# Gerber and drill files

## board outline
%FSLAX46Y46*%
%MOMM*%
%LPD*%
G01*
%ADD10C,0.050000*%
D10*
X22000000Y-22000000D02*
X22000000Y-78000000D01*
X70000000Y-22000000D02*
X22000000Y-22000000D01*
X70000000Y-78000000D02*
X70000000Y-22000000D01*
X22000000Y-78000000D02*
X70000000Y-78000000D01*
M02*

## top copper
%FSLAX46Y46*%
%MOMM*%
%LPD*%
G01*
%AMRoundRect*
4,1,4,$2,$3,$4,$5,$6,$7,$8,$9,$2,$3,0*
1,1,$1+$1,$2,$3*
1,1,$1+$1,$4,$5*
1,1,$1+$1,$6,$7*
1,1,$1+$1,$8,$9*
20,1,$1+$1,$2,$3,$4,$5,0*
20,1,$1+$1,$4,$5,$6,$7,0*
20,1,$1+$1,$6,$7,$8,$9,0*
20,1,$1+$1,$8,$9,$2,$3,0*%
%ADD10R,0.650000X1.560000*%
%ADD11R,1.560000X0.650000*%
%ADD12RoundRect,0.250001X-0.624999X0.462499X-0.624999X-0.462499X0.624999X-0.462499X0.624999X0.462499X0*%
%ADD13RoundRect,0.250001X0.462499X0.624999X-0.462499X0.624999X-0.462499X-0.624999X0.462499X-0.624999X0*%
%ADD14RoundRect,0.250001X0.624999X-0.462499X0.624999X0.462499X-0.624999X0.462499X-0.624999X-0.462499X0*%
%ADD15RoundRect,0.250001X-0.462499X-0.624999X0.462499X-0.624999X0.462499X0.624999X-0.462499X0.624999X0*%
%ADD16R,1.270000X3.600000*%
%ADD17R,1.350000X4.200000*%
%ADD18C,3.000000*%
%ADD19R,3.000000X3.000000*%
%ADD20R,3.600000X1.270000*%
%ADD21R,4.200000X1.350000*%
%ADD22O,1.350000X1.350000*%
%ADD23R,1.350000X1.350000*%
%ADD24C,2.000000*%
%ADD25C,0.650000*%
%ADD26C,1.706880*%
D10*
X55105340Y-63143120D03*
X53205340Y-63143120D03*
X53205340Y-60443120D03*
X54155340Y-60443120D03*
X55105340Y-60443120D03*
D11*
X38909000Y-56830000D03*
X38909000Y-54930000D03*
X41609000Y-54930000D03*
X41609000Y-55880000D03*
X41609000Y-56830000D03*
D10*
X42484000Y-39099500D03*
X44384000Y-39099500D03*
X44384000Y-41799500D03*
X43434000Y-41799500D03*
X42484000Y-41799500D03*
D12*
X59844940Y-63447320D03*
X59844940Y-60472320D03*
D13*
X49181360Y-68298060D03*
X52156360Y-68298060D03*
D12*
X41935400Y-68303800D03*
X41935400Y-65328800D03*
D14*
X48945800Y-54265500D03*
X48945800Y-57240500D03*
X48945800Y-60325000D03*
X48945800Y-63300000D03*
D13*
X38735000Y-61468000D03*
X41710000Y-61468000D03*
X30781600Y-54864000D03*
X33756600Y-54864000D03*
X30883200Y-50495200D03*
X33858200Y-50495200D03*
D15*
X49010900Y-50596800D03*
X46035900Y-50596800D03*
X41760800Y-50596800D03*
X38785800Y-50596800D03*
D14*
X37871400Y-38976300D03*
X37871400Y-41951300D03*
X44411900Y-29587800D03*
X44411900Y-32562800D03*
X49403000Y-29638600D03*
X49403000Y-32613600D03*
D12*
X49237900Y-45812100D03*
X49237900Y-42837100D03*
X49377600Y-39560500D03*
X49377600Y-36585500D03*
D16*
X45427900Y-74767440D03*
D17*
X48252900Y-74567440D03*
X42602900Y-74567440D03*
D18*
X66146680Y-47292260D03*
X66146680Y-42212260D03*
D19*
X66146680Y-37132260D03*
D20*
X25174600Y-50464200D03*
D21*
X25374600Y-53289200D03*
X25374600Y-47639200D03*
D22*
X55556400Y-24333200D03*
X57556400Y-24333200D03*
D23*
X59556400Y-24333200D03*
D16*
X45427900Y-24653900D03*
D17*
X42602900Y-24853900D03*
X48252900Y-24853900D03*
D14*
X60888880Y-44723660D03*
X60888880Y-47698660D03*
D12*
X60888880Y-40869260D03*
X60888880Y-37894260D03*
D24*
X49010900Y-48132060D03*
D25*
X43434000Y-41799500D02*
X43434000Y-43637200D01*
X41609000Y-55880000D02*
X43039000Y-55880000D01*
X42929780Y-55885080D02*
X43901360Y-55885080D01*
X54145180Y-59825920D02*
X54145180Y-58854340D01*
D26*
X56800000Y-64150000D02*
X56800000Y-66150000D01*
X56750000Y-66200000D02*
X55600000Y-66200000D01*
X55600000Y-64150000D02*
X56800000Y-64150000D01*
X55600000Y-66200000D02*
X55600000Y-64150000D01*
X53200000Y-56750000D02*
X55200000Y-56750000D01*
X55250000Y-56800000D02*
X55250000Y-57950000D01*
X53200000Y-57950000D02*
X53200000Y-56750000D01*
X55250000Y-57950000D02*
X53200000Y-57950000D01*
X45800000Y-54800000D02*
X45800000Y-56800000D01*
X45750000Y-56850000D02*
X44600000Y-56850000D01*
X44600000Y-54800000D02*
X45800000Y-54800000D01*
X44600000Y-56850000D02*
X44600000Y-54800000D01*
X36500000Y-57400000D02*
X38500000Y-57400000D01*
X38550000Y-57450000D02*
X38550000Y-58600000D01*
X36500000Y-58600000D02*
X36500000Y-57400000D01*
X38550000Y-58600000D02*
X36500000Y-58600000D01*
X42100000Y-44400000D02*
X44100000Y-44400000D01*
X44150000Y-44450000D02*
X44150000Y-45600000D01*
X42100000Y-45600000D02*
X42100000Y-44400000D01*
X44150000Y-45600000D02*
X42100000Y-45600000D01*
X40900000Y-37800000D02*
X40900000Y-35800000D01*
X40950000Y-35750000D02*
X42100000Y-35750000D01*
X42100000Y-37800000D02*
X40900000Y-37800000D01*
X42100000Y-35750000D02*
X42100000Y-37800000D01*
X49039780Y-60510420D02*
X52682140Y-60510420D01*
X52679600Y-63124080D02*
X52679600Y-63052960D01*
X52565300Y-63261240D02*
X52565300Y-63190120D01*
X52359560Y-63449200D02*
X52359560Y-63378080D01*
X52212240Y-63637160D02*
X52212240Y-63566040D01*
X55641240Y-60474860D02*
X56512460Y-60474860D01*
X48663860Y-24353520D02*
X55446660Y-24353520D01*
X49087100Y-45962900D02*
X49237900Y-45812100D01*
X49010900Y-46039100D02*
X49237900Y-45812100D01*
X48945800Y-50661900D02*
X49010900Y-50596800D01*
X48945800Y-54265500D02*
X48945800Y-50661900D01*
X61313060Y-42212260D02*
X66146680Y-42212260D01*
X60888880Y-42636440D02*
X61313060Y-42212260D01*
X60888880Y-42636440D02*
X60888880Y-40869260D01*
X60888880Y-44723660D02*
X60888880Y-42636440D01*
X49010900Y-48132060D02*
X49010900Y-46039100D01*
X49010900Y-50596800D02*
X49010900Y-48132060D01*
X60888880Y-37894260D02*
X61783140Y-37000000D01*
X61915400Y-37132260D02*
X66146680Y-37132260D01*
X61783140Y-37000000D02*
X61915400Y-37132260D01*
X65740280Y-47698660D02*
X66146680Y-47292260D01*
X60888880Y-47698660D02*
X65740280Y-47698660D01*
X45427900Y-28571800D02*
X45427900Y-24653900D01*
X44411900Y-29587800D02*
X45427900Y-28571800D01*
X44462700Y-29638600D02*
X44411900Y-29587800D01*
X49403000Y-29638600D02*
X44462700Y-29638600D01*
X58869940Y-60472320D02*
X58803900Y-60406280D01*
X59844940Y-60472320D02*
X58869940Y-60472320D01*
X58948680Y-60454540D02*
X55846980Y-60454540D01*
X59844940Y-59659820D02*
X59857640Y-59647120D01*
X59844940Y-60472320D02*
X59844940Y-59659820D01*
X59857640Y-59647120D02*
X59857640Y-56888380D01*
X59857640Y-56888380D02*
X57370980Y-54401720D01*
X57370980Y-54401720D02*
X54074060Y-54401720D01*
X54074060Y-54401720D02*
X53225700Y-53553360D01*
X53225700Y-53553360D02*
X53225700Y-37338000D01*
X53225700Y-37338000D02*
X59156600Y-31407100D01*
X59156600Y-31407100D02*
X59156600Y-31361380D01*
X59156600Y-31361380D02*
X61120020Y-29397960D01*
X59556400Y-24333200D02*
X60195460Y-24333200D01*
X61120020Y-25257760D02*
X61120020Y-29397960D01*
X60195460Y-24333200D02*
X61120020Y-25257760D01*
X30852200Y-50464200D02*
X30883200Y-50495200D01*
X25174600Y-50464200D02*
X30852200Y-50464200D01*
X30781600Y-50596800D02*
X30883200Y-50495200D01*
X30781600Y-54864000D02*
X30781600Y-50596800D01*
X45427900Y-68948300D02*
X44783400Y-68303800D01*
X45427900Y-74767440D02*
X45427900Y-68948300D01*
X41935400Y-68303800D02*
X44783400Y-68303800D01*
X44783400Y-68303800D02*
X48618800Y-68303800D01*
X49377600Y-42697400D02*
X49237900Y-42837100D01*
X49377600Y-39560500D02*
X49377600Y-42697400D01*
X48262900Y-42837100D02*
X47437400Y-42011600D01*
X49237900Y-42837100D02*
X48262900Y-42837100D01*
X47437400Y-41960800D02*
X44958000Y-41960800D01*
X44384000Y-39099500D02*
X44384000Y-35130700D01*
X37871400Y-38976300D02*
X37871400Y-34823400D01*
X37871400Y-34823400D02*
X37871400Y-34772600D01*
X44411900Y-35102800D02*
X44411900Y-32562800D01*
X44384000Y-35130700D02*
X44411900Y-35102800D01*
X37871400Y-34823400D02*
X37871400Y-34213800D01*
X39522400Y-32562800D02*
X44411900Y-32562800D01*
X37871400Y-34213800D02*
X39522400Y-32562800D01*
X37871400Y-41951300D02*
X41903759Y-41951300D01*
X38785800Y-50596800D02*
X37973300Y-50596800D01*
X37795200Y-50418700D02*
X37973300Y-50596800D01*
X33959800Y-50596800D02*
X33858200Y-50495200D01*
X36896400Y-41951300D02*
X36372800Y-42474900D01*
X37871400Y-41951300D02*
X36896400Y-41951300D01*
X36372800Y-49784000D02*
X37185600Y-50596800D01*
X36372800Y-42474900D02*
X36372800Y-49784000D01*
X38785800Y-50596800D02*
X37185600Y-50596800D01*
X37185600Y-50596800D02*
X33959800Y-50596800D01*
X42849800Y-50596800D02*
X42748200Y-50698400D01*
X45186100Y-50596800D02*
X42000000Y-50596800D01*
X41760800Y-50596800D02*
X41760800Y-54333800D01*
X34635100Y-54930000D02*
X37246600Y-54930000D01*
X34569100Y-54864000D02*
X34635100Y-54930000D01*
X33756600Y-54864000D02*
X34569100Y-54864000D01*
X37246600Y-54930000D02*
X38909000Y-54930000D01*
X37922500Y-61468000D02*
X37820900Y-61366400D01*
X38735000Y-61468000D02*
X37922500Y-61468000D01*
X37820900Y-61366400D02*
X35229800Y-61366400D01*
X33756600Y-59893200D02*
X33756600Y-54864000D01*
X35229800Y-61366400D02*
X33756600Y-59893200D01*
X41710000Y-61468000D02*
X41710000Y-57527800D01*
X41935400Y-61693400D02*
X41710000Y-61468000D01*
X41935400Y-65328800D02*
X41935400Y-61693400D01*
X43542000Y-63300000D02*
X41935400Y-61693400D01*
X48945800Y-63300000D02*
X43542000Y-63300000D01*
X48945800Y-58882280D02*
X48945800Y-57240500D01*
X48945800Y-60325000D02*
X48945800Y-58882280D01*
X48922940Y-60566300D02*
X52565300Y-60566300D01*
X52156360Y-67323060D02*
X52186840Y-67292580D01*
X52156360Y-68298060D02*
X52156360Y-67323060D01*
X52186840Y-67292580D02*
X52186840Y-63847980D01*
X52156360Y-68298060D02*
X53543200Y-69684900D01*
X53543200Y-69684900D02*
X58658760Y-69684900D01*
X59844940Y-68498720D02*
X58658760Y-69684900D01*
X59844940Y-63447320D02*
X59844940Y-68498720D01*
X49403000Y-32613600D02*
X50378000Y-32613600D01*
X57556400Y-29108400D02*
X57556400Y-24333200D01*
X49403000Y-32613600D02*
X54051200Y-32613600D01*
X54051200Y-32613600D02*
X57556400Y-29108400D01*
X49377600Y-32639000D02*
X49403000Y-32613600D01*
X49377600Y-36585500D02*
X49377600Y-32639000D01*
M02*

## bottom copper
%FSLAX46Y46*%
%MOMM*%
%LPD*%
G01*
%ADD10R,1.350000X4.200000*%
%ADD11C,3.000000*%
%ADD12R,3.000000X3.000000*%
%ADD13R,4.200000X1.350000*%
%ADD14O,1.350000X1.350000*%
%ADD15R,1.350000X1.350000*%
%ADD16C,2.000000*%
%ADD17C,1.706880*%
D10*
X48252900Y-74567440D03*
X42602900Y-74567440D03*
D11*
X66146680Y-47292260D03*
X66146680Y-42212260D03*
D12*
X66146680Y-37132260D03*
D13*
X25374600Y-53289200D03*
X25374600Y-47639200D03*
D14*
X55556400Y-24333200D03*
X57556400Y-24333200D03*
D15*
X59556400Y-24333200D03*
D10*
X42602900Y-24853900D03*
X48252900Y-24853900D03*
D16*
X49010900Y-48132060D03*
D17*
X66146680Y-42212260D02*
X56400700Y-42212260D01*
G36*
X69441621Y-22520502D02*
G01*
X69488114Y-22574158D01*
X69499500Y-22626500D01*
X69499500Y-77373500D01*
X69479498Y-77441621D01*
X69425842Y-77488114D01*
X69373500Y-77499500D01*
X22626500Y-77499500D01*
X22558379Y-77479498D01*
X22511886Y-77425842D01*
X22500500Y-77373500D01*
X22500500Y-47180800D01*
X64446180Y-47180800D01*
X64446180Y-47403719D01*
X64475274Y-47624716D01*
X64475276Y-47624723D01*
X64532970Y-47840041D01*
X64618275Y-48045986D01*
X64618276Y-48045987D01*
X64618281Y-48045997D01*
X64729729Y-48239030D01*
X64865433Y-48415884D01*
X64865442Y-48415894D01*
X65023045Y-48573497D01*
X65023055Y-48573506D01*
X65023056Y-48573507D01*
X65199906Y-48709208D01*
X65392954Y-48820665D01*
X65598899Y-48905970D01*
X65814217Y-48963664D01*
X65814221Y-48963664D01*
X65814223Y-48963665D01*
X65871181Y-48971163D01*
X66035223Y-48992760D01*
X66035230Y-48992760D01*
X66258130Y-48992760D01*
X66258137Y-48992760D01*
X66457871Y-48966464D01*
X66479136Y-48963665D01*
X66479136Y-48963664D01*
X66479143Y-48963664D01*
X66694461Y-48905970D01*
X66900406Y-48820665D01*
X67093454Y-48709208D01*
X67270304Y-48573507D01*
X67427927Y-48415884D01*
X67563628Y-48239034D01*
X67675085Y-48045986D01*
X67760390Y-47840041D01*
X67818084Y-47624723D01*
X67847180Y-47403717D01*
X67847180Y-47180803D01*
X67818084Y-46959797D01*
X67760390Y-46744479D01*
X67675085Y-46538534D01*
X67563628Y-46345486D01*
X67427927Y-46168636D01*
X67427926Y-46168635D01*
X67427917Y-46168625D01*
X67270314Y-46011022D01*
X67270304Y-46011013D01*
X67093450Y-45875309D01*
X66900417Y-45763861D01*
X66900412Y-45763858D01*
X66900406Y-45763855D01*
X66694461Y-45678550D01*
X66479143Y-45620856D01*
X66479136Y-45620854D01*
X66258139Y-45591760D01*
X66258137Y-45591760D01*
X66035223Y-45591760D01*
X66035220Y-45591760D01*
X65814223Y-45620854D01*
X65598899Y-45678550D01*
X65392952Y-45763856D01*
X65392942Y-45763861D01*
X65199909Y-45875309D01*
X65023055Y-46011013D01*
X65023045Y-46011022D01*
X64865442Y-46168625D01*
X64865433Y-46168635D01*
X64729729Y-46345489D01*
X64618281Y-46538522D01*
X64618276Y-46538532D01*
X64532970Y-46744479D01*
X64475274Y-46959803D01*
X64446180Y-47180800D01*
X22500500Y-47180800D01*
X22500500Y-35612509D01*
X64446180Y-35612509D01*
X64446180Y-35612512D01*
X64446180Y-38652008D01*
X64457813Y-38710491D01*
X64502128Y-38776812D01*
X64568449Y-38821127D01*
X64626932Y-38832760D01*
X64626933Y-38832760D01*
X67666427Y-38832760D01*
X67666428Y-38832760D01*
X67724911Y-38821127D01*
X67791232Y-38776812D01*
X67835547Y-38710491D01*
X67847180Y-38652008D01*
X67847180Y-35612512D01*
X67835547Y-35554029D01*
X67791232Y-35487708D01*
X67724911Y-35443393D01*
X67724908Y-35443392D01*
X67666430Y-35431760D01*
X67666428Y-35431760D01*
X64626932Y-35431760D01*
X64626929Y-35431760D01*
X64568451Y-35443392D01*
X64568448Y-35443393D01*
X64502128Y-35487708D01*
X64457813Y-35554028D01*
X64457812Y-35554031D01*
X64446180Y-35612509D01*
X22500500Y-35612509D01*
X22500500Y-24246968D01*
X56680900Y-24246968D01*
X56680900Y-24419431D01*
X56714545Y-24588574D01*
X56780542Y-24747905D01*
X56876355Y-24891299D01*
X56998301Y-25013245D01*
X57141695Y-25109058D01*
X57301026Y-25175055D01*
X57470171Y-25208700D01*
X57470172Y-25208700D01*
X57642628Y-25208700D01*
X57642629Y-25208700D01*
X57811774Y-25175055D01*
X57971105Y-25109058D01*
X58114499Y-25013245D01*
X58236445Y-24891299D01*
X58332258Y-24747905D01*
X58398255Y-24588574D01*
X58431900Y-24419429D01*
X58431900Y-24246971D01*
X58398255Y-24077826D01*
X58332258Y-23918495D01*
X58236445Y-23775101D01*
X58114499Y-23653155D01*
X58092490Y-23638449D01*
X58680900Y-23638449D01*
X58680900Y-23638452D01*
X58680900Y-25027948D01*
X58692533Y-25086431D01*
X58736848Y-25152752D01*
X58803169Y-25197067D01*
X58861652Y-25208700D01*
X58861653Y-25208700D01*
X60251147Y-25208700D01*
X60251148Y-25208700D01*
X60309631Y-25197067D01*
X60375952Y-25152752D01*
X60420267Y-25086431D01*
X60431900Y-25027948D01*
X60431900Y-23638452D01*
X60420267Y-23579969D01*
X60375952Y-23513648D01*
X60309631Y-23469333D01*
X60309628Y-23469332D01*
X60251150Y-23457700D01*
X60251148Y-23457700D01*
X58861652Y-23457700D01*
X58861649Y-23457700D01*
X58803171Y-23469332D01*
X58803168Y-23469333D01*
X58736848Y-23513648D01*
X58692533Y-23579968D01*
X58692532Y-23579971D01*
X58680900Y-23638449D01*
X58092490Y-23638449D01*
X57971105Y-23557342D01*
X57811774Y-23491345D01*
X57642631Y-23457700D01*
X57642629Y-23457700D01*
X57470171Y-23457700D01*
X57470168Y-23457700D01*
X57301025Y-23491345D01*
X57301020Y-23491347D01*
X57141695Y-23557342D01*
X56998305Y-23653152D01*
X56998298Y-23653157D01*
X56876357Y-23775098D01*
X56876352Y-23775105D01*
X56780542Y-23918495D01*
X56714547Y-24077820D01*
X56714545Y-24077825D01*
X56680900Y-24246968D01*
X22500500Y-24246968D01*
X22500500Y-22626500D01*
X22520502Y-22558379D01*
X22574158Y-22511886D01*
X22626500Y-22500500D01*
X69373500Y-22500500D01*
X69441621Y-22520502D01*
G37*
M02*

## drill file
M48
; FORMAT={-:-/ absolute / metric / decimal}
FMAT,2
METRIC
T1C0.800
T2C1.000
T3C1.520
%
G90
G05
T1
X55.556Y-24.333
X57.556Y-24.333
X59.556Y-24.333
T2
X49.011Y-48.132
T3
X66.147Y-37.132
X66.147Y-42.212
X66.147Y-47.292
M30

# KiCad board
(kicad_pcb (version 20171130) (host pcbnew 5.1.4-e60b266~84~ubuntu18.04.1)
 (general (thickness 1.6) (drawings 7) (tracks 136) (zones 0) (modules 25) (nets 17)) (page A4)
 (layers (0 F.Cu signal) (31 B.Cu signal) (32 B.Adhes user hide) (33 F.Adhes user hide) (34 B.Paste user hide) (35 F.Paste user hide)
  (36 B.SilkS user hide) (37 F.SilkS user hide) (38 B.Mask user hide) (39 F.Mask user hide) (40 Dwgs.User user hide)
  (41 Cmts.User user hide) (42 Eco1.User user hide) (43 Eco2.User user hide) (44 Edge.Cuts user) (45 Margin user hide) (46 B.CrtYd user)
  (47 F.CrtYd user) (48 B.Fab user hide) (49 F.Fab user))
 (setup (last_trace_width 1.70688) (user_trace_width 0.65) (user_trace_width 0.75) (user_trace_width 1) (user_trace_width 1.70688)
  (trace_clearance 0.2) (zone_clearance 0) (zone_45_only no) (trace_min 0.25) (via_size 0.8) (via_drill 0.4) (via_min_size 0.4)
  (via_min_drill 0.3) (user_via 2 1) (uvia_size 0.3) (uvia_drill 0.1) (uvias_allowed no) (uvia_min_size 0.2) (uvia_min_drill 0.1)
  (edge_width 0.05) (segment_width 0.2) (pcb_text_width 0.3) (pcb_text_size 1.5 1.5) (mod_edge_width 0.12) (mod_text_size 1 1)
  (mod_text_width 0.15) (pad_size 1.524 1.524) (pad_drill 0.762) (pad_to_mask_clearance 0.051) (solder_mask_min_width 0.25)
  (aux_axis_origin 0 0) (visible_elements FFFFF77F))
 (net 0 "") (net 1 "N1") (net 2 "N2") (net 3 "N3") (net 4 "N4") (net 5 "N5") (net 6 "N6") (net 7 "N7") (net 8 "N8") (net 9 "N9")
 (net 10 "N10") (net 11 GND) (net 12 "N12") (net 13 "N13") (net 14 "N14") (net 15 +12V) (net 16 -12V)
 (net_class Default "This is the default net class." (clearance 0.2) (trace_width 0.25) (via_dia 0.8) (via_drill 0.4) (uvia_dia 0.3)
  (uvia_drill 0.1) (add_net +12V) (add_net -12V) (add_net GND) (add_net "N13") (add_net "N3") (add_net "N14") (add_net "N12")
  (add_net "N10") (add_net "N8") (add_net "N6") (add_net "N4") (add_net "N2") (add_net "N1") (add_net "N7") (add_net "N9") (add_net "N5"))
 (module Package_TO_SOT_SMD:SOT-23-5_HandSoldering (layer F.Cu) (at 54.15534 61.79312 270)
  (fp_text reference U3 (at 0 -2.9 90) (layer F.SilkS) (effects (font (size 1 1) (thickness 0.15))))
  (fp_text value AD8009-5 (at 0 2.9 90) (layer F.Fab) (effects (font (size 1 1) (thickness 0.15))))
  (pad 5 smd rect (at 1.35 -0.95 270) (size 1.56 0.65) (layers F.Cu F.Paste F.Mask))
  (pad 4 smd rect (at 1.35 0.95 270) (size 1.56 0.65) (layers F.Cu F.Paste F.Mask) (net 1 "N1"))
  (pad 3 smd rect (at -1.35 0.95 270) (size 1.56 0.65) (layers F.Cu F.Paste F.Mask) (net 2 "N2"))
  (pad 2 smd rect (at -1.35 0 270) (size 1.56 0.65) (layers F.Cu F.Paste F.Mask))
  (pad 1 smd rect (at -1.35 -0.95 270) (size 1.56 0.65) (layers F.Cu F.Paste F.Mask) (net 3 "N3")))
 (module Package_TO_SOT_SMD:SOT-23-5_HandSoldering (layer F.Cu) (at 40.259 55.88 180)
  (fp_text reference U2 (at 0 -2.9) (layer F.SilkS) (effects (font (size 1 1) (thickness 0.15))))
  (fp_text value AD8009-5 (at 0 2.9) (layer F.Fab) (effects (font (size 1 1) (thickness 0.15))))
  (pad 5 smd rect (at 1.35 -0.95 180) (size 1.56 0.65) (layers F.Cu F.Paste F.Mask))
  (pad 4 smd rect (at 1.35 0.95 180) (size 1.56 0.65) (layers F.Cu F.Paste F.Mask) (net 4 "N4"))
  (pad 3 smd rect (at -1.35 0.95 180) (size 1.56 0.65) (layers F.Cu F.Paste F.Mask) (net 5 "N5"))
  (pad 2 smd rect (at -1.35 0 180) (size 1.56 0.65) (layers F.Cu F.Paste F.Mask))
  (pad 1 smd rect (at -1.35 -0.95 180) (size 1.56 0.65) (layers F.Cu F.Paste F.Mask) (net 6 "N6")))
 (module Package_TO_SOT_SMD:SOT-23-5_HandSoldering (layer F.Cu) (at 43.434 40.4495 90)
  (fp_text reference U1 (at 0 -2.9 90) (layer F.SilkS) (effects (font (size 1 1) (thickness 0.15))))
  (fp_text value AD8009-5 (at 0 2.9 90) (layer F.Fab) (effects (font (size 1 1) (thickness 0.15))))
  (pad 5 smd rect (at 1.35 -0.95 90) (size 1.56 0.65) (layers F.Cu F.Paste F.Mask))
  (pad 4 smd rect (at 1.35 0.95 90) (size 1.56 0.65) (layers F.Cu F.Paste F.Mask) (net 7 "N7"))
  (pad 3 smd rect (at -1.35 0.95 90) (size 1.56 0.65) (layers F.Cu F.Paste F.Mask) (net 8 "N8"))
  (pad 2 smd rect (at -1.35 0 90) (size 1.56 0.65) (layers F.Cu F.Paste F.Mask))
  (pad 1 smd rect (at -1.35 -0.95 90) (size 1.56 0.65) (layers F.Cu F.Paste F.Mask) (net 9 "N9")))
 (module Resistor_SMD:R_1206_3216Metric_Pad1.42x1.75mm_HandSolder (layer F.Cu) (at 59.84494 61.95982 270)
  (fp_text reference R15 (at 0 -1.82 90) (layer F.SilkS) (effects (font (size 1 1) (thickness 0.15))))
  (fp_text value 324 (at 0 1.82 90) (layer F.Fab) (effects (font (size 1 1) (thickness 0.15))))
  (pad 2 smd roundrect (at 1.4875 0 270) (size 1.425 1.75) (layers F.Cu F.Paste F.Mask) (roundrect_rratio 0.175439) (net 1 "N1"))
  (pad 1 smd roundrect (at -1.4875 0 270) (size 1.425 1.75) (layers F.Cu F.Paste F.Mask) (roundrect_rratio 0.175439) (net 3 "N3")))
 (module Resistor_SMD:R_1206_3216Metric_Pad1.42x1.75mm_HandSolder (layer F.Cu) (at 50.66886 68.29806 180)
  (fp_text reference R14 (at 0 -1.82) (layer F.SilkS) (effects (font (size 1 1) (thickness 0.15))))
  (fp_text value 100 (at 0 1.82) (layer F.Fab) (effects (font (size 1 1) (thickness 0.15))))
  (pad 2 smd roundrect (at 1.4875 0 180) (size 1.425 1.75) (layers F.Cu F.Paste F.Mask) (roundrect_rratio 0.175439) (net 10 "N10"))
  (pad 1 smd roundrect (at -1.4875 0 180) (size 1.425 1.75) (layers F.Cu F.Paste F.Mask) (roundrect_rratio 0.175439) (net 1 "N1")))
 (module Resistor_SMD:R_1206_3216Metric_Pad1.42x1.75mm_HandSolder (layer F.Cu) (at 41.9354 66.8163 270)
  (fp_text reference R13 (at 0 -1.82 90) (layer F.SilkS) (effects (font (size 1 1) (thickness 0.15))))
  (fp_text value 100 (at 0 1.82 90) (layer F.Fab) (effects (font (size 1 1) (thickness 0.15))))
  (pad 2 smd roundrect (at 1.4875 0 270) (size 1.425 1.75) (layers F.Cu F.Paste F.Mask) (roundrect_rratio 0.175439) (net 10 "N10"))
  (pad 1 smd roundrect (at -1.4875 0 270) (size 1.425 1.75) (layers F.Cu F.Paste F.Mask) (roundrect_rratio 0.175439) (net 6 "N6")))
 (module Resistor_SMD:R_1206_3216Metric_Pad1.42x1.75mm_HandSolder (layer F.Cu) (at 48.9458 55.753 90)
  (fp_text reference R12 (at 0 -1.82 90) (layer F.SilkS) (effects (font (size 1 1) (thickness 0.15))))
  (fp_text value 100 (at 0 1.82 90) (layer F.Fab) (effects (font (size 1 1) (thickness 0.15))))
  (pad 2 smd roundrect (at 1.4875 0 90) (size 1.425 1.75) (layers F.Cu F.Paste F.Mask) (roundrect_rratio 0.175439) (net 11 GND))
  (pad 1 smd roundrect (at -1.4875 0 90) (size 1.425 1.75) (layers F.Cu F.Paste F.Mask) (roundrect_rratio 0.175439) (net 2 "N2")))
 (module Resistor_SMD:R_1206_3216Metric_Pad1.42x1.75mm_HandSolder (layer F.Cu) (at 48.9458 61.8125 90)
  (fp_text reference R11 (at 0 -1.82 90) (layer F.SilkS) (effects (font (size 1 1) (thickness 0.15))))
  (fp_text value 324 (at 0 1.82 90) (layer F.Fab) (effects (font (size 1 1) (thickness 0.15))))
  (pad 2 smd roundrect (at 1.4875 0 90) (size 1.425 1.75) (layers F.Cu F.Paste F.Mask) (roundrect_rratio 0.175439) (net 2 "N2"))
  (pad 1 smd roundrect (at -1.4875 0 90) (size 1.425 1.75) (layers F.Cu F.Paste F.Mask) (roundrect_rratio 0.175439) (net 6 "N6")))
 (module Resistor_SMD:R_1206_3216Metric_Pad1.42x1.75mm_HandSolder (layer F.Cu) (at 40.2225 61.468 180)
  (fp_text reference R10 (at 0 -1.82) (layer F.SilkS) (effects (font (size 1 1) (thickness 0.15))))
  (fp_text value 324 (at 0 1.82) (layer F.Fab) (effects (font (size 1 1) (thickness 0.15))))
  (pad 2 smd roundrect (at 1.4875 0 180) (size 1.425 1.75) (layers F.Cu F.Paste F.Mask) (roundrect_rratio 0.175439) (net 4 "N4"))
  (pad 1 smd roundrect (at -1.4875 0 180) (size 1.425 1.75) (layers F.Cu F.Paste F.Mask) (roundrect_rratio 0.175439) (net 6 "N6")))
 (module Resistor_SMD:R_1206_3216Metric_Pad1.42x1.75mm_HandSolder (layer F.Cu) (at 32.2691 54.864 180)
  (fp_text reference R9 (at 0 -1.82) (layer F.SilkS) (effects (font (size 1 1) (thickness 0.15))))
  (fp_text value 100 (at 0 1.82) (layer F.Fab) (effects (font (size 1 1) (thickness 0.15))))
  (pad 2 smd roundrect (at 1.4875 0 180) (size 1.425 1.75) (layers F.Cu F.Paste F.Mask) (roundrect_rratio 0.175439) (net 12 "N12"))
  (pad 1 smd roundrect (at -1.4875 0 180) (size 1.425 1.75) (layers F.Cu F.Paste F.Mask) (roundrect_rratio 0.175439) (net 4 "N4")))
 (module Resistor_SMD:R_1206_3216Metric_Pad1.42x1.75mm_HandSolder (layer F.Cu) (at 32.3707 50.4952 180)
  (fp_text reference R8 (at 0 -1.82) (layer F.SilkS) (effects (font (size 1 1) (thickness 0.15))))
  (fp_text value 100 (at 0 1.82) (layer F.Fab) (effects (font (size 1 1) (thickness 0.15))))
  (pad 2 smd roundrect (at 1.4875 0 180) (size 1.425 1.75) (layers F.Cu F.Paste F.Mask) (roundrect_rratio 0.175439) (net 12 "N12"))
  (pad 1 smd roundrect (at -1.4875 0 180) (size 1.425 1.75) (layers F.Cu F.Paste F.Mask) (roundrect_rratio 0.175439) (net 9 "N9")))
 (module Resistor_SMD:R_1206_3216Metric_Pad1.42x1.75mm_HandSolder (layer F.Cu) (at 47.5234 50.5968)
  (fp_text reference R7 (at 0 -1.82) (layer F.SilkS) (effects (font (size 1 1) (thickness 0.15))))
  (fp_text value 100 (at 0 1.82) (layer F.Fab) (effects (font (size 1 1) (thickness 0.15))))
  (pad 2 smd roundrect (at 1.4875 0) (size 1.425 1.75) (layers F.Cu F.Paste F.Mask) (roundrect_rratio 0.175439) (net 11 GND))
  (pad 1 smd roundrect (at -1.4875 0) (size 1.425 1.75) (layers F.Cu F.Paste F.Mask) (roundrect_rratio 0.175439) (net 5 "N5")))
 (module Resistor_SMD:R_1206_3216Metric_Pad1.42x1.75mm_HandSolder (layer F.Cu) (at 40.2733 50.5968)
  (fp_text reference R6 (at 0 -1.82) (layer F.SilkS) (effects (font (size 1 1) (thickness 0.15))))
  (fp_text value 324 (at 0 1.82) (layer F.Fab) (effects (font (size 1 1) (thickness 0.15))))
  (pad 2 smd roundrect (at 1.4875 0) (size 1.425 1.75) (layers F.Cu F.Paste F.Mask) (roundrect_rratio 0.175439) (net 5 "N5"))
  (pad 1 smd roundrect (at -1.4875 0) (size 1.425 1.75) (layers F.Cu F.Paste F.Mask) (roundrect_rratio 0.175439) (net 9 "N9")))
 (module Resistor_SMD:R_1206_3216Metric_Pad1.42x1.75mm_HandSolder (layer F.Cu) (at 37.8714 40.4638 90)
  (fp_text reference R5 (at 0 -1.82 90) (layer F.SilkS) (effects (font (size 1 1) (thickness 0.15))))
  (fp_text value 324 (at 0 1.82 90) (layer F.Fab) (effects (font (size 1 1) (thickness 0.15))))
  (pad 2 smd roundrect (at 1.4875 0 90) (size 1.425 1.75) (layers F.Cu F.Paste F.Mask) (roundrect_rratio 0.175439) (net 7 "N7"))
  (pad 1 smd roundrect (at -1.4875 0 90) (size 1.425 1.75) (layers F.Cu F.Paste F.Mask) (roundrect_rratio 0.175439) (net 9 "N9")))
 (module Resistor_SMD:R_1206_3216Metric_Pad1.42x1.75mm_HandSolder (layer F.Cu) (at 44.4119 31.0753 90)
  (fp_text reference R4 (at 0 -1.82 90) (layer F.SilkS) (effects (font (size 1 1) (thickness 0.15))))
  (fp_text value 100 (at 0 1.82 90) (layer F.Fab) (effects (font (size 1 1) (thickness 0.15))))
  (pad 2 smd roundrect (at 1.4875 0 90) (size 1.425 1.75) (layers F.Cu F.Paste F.Mask) (roundrect_rratio 0.175439) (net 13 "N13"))
  (pad 1 smd roundrect (at -1.4875 0 90) (size 1.425 1.75) (layers F.Cu F.Paste F.Mask) (roundrect_rratio 0.175439) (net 7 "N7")))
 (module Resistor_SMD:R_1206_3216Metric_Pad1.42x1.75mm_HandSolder (layer F.Cu) (at 49.403 31.1261 90)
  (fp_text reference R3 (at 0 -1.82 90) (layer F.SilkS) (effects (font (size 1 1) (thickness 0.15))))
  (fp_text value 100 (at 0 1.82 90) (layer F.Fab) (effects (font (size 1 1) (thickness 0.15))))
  (pad 2 smd roundrect (at 1.4875 0 90) (size 1.425 1.75) (layers F.Cu F.Paste F.Mask) (roundrect_rratio 0.175439) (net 13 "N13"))
  (pad 1 smd roundrect (at -1.4875 0 90) (size 1.425 1.75) (layers F.Cu F.Paste F.Mask) (roundrect_rratio 0.175439) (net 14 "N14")))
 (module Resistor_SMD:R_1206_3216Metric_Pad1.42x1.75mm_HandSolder (layer F.Cu) (at 49.2379 44.3246 270)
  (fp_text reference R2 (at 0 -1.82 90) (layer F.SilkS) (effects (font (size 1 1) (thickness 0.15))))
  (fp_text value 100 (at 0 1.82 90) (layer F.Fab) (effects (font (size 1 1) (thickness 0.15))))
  (pad 2 smd roundrect (at 1.4875 0 270) (size 1.425 1.75) (layers F.Cu F.Paste F.Mask) (roundrect_rratio 0.175439) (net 11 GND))
  (pad 1 smd roundrect (at -1.4875 0 270) (size 1.425 1.75) (layers F.Cu F.Paste F.Mask) (roundrect_rratio 0.175439) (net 8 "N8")))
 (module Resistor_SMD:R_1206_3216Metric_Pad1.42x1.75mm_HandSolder (layer F.Cu) (at 49.3776 38.073 270)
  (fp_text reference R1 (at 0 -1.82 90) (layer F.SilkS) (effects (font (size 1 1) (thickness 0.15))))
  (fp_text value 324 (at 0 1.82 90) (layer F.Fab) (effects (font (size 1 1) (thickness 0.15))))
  (pad 2 smd roundrect (at 1.4875 0 270) (size 1.425 1.75) (layers F.Cu F.Paste F.Mask) (roundrect_rratio 0.175439) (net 8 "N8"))
  (pad 1 smd roundrect (at -1.4875 0 270) (size 1.425 1.75) (layers F.Cu F.Paste F.Mask) (roundrect_rratio 0.175439) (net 14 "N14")))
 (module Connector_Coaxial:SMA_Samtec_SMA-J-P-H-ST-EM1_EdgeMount (layer F.Cu) (at 45.4279 74.56744 270)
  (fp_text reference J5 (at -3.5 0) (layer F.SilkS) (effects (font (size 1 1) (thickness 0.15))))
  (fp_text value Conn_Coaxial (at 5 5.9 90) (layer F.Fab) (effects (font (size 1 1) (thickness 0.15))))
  (pad 1 smd rect (at 0.2 0) (size 1.27 3.6) (layers F.Cu F.Paste F.Mask) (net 10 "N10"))
  (pad 2 smd rect (at 0 -2.825) (size 1.35 4.2) (layers F.Cu F.Paste F.Mask) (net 11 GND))
  (pad 2 smd rect (at 0 2.825) (size 1.35 4.2) (layers F.Cu F.Paste F.Mask) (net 11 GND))
  (pad 2 smd rect (at 0 -2.825) (size 1.35 4.2) (layers B.Cu B.Paste B.Mask) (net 11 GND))
  (pad 2 smd rect (at 0 2.825) (size 1.35 4.2) (layers B.Cu B.Paste B.Mask) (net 11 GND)))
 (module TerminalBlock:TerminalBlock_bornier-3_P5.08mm (layer F.Cu) (at 66.14668 37.13226 270)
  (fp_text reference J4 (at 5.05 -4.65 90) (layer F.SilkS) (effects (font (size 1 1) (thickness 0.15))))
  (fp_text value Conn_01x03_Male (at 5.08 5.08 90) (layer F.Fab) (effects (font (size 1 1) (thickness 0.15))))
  (pad 3 thru_hole circle (at 10.16 0 270) (size 3 3) (drill 1.52) (layers *.Cu *.Mask) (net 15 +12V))
  (pad 2 thru_hole circle (at 5.08 0 270) (size 3 3) (drill 1.52) (layers *.Cu *.Mask) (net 11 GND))
  (pad 1 thru_hole rect (at 0 0 270) (size 3 3) (drill 1.52) (layers *.Cu *.Mask) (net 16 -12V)))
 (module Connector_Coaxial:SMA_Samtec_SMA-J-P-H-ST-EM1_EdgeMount (layer F.Cu) (at 25.3746 50.4642 180)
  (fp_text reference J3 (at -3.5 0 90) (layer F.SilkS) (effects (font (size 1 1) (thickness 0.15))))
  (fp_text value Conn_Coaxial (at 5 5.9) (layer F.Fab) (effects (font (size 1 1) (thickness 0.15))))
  (pad 1 smd rect (at 0.2 0 270) (size 1.27 3.6) (layers F.Cu F.Paste F.Mask) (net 12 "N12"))
  (pad 2 smd rect (at 0 -2.825 270) (size 1.35 4.2) (layers F.Cu F.Paste F.Mask) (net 11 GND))
  (pad 2 smd rect (at 0 2.825 270) (size 1.35 4.2) (layers F.Cu F.Paste F.Mask) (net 11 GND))
  (pad 2 smd rect (at 0 -2.825 270) (size 1.35 4.2) (layers B.Cu B.Paste B.Mask) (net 11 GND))
  (pad 2 smd rect (at 0 2.825 270) (size 1.35 4.2) (layers B.Cu B.Paste B.Mask) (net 11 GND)))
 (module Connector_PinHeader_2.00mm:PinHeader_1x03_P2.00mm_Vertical (layer F.Cu) (at 59.5564 24.3332 270)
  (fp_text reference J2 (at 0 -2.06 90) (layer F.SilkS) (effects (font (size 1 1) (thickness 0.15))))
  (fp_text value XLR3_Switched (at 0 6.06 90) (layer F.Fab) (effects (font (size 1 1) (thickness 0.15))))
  (pad 3 thru_hole oval (at 0 4 270) (size 1.35 1.35) (drill 0.8) (layers *.Cu *.Mask) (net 11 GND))
  (pad 2 thru_hole oval (at 0 2 270) (size 1.35 1.35) (drill 0.8) (layers *.Cu *.Mask) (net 14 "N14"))
  (pad 1 thru_hole rect (at 0 0 270) (size 1.35 1.35) (drill 0.8) (layers *.Cu *.Mask) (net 3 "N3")))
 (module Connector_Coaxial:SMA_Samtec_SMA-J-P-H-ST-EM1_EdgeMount (layer F.Cu) (at 45.4279 24.8539 90)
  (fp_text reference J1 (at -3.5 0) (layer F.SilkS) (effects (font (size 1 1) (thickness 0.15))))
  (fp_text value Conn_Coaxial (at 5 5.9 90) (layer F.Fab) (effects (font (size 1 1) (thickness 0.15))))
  (pad 1 smd rect (at 0.2 0 180) (size 1.27 3.6) (layers F.Cu F.Paste F.Mask) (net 13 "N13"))
  (pad 2 smd rect (at 0 -2.825 180) (size 1.35 4.2) (layers F.Cu F.Paste F.Mask) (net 11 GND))
  (pad 2 smd rect (at 0 2.825 180) (size 1.35 4.2) (layers F.Cu F.Paste F.Mask) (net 11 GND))
  (pad 2 smd rect (at 0 -2.825 180) (size 1.35 4.2) (layers B.Cu B.Paste B.Mask) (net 11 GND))
  (pad 2 smd rect (at 0 2.825 180) (size 1.35 4.2) (layers B.Cu B.Paste B.Mask) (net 11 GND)))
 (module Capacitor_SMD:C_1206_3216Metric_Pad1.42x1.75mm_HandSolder (layer F.Cu) (at 60.88888 46.21116 90)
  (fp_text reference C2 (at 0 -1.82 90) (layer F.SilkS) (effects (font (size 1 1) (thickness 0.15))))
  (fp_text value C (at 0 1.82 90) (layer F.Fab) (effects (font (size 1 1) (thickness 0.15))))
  (pad 2 smd roundrect (at 1.4875 0 90) (size 1.425 1.75) (layers F.Cu F.Paste F.Mask) (roundrect_rratio 0.175439) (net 11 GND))
  (pad 1 smd roundrect (at -1.4875 0 90) (size 1.425 1.75) (layers F.Cu F.Paste F.Mask) (roundrect_rratio 0.175439) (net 15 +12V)))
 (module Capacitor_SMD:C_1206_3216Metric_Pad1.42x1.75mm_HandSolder (layer F.Cu) (at 60.88888 39.38176 270)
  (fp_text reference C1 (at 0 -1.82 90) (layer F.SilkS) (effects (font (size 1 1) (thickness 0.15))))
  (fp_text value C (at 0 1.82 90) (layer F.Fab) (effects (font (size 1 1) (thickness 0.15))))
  (pad 2 smd roundrect (at 1.4875 0 270) (size 1.425 1.75) (layers F.Cu F.Paste F.Mask) (roundrect_rratio 0.175439) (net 11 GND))
  (pad 1 smd roundrect (at -1.4875 0 270) (size 1.425 1.75) (layers F.Cu F.Paste F.Mask) (roundrect_rratio 0.175439) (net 16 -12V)))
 (gr_line (start 22 22) (end 22 78) (layer Edge.Cuts) (width 0.05))
 (gr_line (start 70 22) (end 22 22) (layer Edge.Cuts) (width 0.05))
 (gr_line (start 70 78) (end 70 22) (layer Edge.Cuts) (width 0.05))
 (gr_line (start 22 78) (end 70 78) (layer Edge.Cuts) (width 0.05))
 (segment (start 43.434 41.7995) (end 43.434 43.6372) (width 0.65) (layer F.Cu) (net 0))
 (segment (start 41.609 55.88) (end 43.039 55.88) (width 0.65) (layer F.Cu) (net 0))
 (segment (start 42.92978 55.88508) (end 43.90136 55.88508) (width 0.65) (layer F.Cu) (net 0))
 (segment (start 54.14518 59.82592) (end 54.14518 58.85434) (width 0.65) (layer F.Cu) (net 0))
 (segment (start 56.8 64.15) (end 56.8 66.15) (width 1.70688) (layer F.Cu) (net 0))
 (segment (start 56.75 66.2) (end 55.6 66.2) (width 1.70688) (layer F.Cu) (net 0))
 (segment (start 55.6 64.15) (end 56.8 64.15) (width 1.70688) (layer F.Cu) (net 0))
 (segment (start 55.6 66.2) (end 55.6 64.15) (width 1.70688) (layer F.Cu) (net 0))
 (segment (start 53.2 56.75) (end 55.2 56.75) (width 1.70688) (layer F.Cu) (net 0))
 (segment (start 55.25 56.8) (end 55.25 57.95) (width 1.70688) (layer F.Cu) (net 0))
 (segment (start 53.2 57.95) (end 53.2 56.75) (width 1.70688) (layer F.Cu) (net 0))
 (segment (start 55.25 57.95) (end 53.2 57.95) (width 1.70688) (layer F.Cu) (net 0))
 (segment (start 45.8 54.8) (end 45.8 56.8) (width 1.70688) (layer F.Cu) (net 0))
 (segment (start 45.75 56.85) (end 44.6 56.85) (width 1.70688) (layer F.Cu) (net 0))
 (segment (start 44.6 54.8) (end 45.8 54.8) (width 1.70688) (layer F.Cu) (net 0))
 (segment (start 44.6 56.85) (end 44.6 54.8) (width 1.70688) (layer F.Cu) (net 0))
 (segment (start 36.5 57.4) (end 38.5 57.4) (width 1.70688) (layer F.Cu) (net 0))
 (segment (start 38.55 57.45) (end 38.55 58.6) (width 1.70688) (layer F.Cu) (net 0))
 (segment (start 36.5 58.6) (end 36.5 57.4) (width 1.70688) (layer F.Cu) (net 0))
 (segment (start 38.55 58.6) (end 36.5 58.6) (width 1.70688) (layer F.Cu) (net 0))
 (segment (start 42.1 44.4) (end 44.1 44.4) (width 1.70688) (layer F.Cu) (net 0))
 (segment (start 44.15 44.45) (end 44.15 45.6) (width 1.70688) (layer F.Cu) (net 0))
 (segment (start 42.1 45.6) (end 42.1 44.4) (width 1.70688) (layer F.Cu) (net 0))
 (segment (start 44.15 45.6) (end 42.1 45.6) (width 1.70688) (layer F.Cu) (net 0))
 (segment (start 40.9 37.8) (end 40.9 35.8) (width 1.70688) (layer F.Cu) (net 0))
 (segment (start 40.95 35.75) (end 42.1 35.75) (width 1.70688) (layer F.Cu) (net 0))
 (segment (start 42.1 37.8) (end 40.9 37.8) (width 1.70688) (layer F.Cu) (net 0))
 (segment (start 42.1 35.75) (end 42.1 37.8) (width 1.70688) (layer F.Cu) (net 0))
 (segment (start 49.03978 60.51042) (end 52.68214 60.51042) (width 1.70688) (layer F.Cu) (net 2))
 (segment (start 52.6796 63.12408) (end 52.6796 63.05296) (width 1.70688) (layer F.Cu) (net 1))
 (segment (start 52.5653 63.26124) (end 52.5653 63.19012) (width 1.70688) (layer F.Cu) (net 1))
 (segment (start 52.35956 63.4492) (end 52.35956 63.37808) (width 1.70688) (layer F.Cu) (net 1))
 (segment (start 52.21224 63.63716) (end 52.21224 63.56604) (width 1.70688) (layer F.Cu) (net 1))
 (segment (start 55.64124 60.47486) (end 56.51246 60.47486) (width 1.70688) (layer F.Cu) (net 3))
 (segment (start 48.66386 24.35352) (end 55.44666 24.35352) (width 1.70688) (layer F.Cu) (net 11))
 (segment (start 49.0871 45.9629) (end 49.2379 45.8121) (width 1.70688) (layer F.Cu) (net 11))
 (segment (start 49.0109 46.0391) (end 49.2379 45.8121) (width 1.70688) (layer F.Cu) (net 11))
 (segment (start 48.9458 50.6619) (end 49.0109 50.5968) (width 1.70688) (layer F.Cu) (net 11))
 (segment (start 48.9458 54.2655) (end 48.9458 50.6619) (width 1.70688) (layer F.Cu) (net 11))
 (segment (start 61.31306 42.21226) (end 66.14668 42.21226) (width 1.70688) (layer F.Cu) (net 11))
 (segment (start 60.88888 42.63644) (end 61.31306 42.21226) (width 1.70688) (layer F.Cu) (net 11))
 (segment (start 60.88888 42.63644) (end 60.88888 40.86926) (width 1.70688) (layer F.Cu) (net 11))
 (segment (start 60.88888 44.72366) (end 60.88888 42.63644) (width 1.70688) (layer F.Cu) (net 11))
 (segment (start 66.14668 42.21226) (end 56.4007 42.21226) (width 1.70688) (layer B.Cu) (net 11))
 (via (at 49.0109 48.13206) (size 2) (drill 1) (layers F.Cu B.Cu) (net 11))
 (segment (start 49.0109 48.13206) (end 49.0109 46.0391) (width 1.70688) (layer F.Cu) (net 11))
 (segment (start 49.0109 50.5968) (end 49.0109 48.13206) (width 1.70688) (layer F.Cu) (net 11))
 (segment (start 60.88888 37.89426) (end 61.78314 37) (width 1.70688) (layer F.Cu) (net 16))
 (segment (start 61.9154 37.13226) (end 66.14668 37.13226) (width 1.70688) (layer F.Cu) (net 16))
 (segment (start 61.78314 37) (end 61.9154 37.13226) (width 1.70688) (layer F.Cu) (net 16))
 (segment (start 65.74028 47.69866) (end 66.14668 47.29226) (width 1.70688) (layer F.Cu) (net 15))
 (segment (start 60.88888 47.69866) (end 65.74028 47.69866) (width 1.70688) (layer F.Cu) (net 15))
 (segment (start 45.4279 28.5718) (end 45.4279 24.6539) (width 1.70688) (layer F.Cu) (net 13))
 (segment (start 44.4119 29.5878) (end 45.4279 28.5718) (width 1.70688) (layer F.Cu) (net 13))
 (segment (start 44.4627 29.6386) (end 44.4119 29.5878) (width 1.70688) (layer F.Cu) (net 13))
 (segment (start 49.403 29.6386) (end 44.4627 29.6386) (width 1.70688) (layer F.Cu) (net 13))
 (segment (start 58.86994 60.47232) (end 58.8039 60.40628) (width 1.70688) (layer F.Cu) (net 3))
 (segment (start 59.84494 60.47232) (end 58.86994 60.47232) (width 1.70688) (layer F.Cu) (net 3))
 (segment (start 58.94868 60.45454) (end 55.84698 60.45454) (width 1.70688) (layer F.Cu) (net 3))
 (segment (start 59.84494 59.65982) (end 59.85764 59.64712) (width 1.70688) (layer F.Cu) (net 3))
 (segment (start 59.84494 60.47232) (end 59.84494 59.65982) (width 1.70688) (layer F.Cu) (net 3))
 (segment (start 59.85764 59.64712) (end 59.85764 56.88838) (width 1.70688) (layer F.Cu) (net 3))
 (segment (start 59.85764 56.88838) (end 57.37098 54.40172) (width 1.70688) (layer F.Cu) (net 3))
 (segment (start 57.37098 54.40172) (end 54.07406 54.40172) (width 1.70688) (layer F.Cu) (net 3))
 (segment (start 54.07406 54.40172) (end 53.2257 53.55336) (width 1.70688) (layer F.Cu) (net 3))
 (segment (start 53.2257 53.55336) (end 53.2257 37.338) (width 1.70688) (layer F.Cu) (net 3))
 (segment (start 53.2257 37.338) (end 59.1566 31.4071) (width 1.70688) (layer F.Cu) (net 3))
 (segment (start 59.1566 31.4071) (end 59.1566 31.36138) (width 1.70688) (layer F.Cu) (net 3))
 (segment (start 59.1566 31.36138) (end 61.12002 29.39796) (width 1.70688) (layer F.Cu) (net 3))
 (segment (start 59.5564 24.3332) (end 60.19546 24.3332) (width 1.70688) (layer F.Cu) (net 3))
 (segment (start 61.12002 25.25776) (end 61.12002 29.39796) (width 1.70688) (layer F.Cu) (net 3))
 (segment (start 60.19546 24.3332) (end 61.12002 25.25776) (width 1.70688) (layer F.Cu) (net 3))
 (segment (start 30.8522 50.4642) (end 30.8832 50.4952) (width 1.70688) (layer F.Cu) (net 12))
 (segment (start 25.1746 50.4642) (end 30.8522 50.4642) (width 1.70688) (layer F.Cu) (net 12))
 (segment (start 30.7816 50.5968) (end 30.8832 50.4952) (width 1.70688) (layer F.Cu) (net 12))
 (segment (start 30.7816 54.864) (end 30.7816 50.5968) (width 1.70688) (layer F.Cu) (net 12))
 (segment (start 45.4279 68.9483) (end 44.7834 68.3038) (width 1.70688) (layer F.Cu) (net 10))
 (segment (start 45.4279 74.76744) (end 45.4279 68.9483) (width 1.70688) (layer F.Cu) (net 10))
 (segment (start 41.9354 68.3038) (end 44.7834 68.3038) (width 1.70688) (layer F.Cu) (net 10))
 (segment (start 44.7834 68.3038) (end 48.6188 68.3038) (width 1.70688) (layer F.Cu) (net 10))
 (segment (start 49.3776 42.6974) (end 49.2379 42.8371) (width 1.70688) (layer F.Cu) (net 8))
 (segment (start 49.3776 39.5605) (end 49.3776 42.6974) (width 1.70688) (layer F.Cu) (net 8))
 (segment (start 48.2629 42.8371) (end 47.4374 42.0116) (width 1.70688) (layer F.Cu) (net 8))
 (segment (start 49.2379 42.8371) (end 48.2629 42.8371) (width 1.70688) (layer F.Cu) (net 8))
 (segment (start 47.4374 41.9608) (end 44.958 41.9608) (width 1.70688) (layer F.Cu) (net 8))
 (segment (start 44.384 39.0995) (end 44.384 35.1307) (width 1.70688) (layer F.Cu) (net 7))
 (segment (start 37.8714 38.9763) (end 37.8714 34.8234) (width 1.70688) (layer F.Cu) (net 7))
 (segment (start 37.8714 34.8234) (end 37.8714 34.7726) (width 1.70688) (layer F.Cu) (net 7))
 (segment (start 44.4119 35.1028) (end 44.4119 32.5628) (width 1.70688) (layer F.Cu) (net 7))
 (segment (start 44.384 35.1307) (end 44.4119 35.1028) (width 1.70688) (layer F.Cu) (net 7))
 (segment (start 37.8714 34.8234) (end 37.8714 34.2138) (width 1.70688) (layer F.Cu) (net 7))
 (segment (start 39.5224 32.5628) (end 44.4119 32.5628) (width 1.70688) (layer F.Cu) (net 7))
 (segment (start 37.8714 34.2138) (end 39.5224 32.5628) (width 1.70688) (layer F.Cu) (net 7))
 (segment (start 37.8714 41.9513) (end 41.903759 41.9513) (width 1.70688) (layer F.Cu) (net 9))
 (segment (start 38.7858 50.5968) (end 37.9733 50.5968) (width 1.70688) (layer F.Cu) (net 9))
 (segment (start 37.7952 50.4187) (end 37.9733 50.5968) (width 1.70688) (layer F.Cu) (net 9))
 (segment (start 33.9598 50.5968) (end 33.8582 50.4952) (width 1.70688) (layer F.Cu) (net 9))
 (segment (start 36.8964 41.9513) (end 36.3728 42.4749) (width 1.70688) (layer F.Cu) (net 9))
 (segment (start 37.8714 41.9513) (end 36.8964 41.9513) (width 1.70688) (layer F.Cu) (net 9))
 (segment (start 36.3728 49.784) (end 37.1856 50.5968) (width 1.70688) (layer F.Cu) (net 9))
 (segment (start 36.3728 42.4749) (end 36.3728 49.784) (width 1.70688) (layer F.Cu) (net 9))
 (segment (start 38.7858 50.5968) (end 37.1856 50.5968) (width 1.70688) (layer F.Cu) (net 9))
 (segment (start 37.1856 50.5968) (end 33.9598 50.5968) (width 1.70688) (layer F.Cu) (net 9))
 (segment (start 42.8498 50.5968) (end 42.7482 50.6984) (width 1.70688) (layer F.Cu) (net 5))
 (segment (start 45.1861 50.5968) (end 42 50.5968) (width 1.70688) (layer F.Cu) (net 5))
 (segment (start 41.7608 50.5968) (end 41.7608 54.3338) (width 1.70688) (layer F.Cu) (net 5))
 (segment (start 34.6351 54.93) (end 37.2466 54.93) (width 1.70688) (layer F.Cu) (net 4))
 (segment (start 34.5691 54.864) (end 34.6351 54.93) (width 1.70688) (layer F.Cu) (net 4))
 (segment (start 33.7566 54.864) (end 34.5691 54.864) (width 1.70688) (layer F.Cu) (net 4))
 (segment (start 37.2466 54.93) (end 38.909 54.93) (width 1.70688) (layer F.Cu) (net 4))
 (segment (start 37.9225 61.468) (end 37.8209 61.3664) (width 1.70688) (layer F.Cu) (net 4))
 (segment (start 38.735 61.468) (end 37.9225 61.468) (width 1.70688) (layer F.Cu) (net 4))
 (segment (start 37.8209 61.3664) (end 35.2298 61.3664) (width 1.70688) (layer F.Cu) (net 4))
 (segment (start 33.7566 59.8932) (end 33.7566 54.864) (width 1.70688) (layer F.Cu) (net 4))
 (segment (start 35.2298 61.3664) (end 33.7566 59.8932) (width 1.70688) (layer F.Cu) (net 4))
 (segment (start 41.71 61.468) (end 41.71 57.5278) (width 1.70688) (layer F.Cu) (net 6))
 (segment (start 41.9354 61.6934) (end 41.71 61.468) (width 1.70688) (layer F.Cu) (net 6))
 (segment (start 41.9354 65.3288) (end 41.9354 61.6934) (width 1.70688) (layer F.Cu) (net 6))
 (segment (start 43.542 63.3) (end 41.9354 61.6934) (width 1.70688) (layer F.Cu) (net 6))
 (segment (start 48.9458 63.3) (end 43.542 63.3) (width 1.70688) (layer F.Cu) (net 6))
 (segment (start 48.9458 58.88228) (end 48.9458 57.2405) (width 1.70688) (layer F.Cu) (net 2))
 (segment (start 48.9458 60.325) (end 48.9458 58.88228) (width 1.70688) (layer F.Cu) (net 2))
 (segment (start 48.92294 60.5663) (end 52.5653 60.5663) (width 1.70688) (layer F.Cu) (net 2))
 (segment (start 52.15636 67.32306) (end 52.18684 67.29258) (width 1.70688) (layer F.Cu) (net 1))
 (segment (start 52.15636 68.29806) (end 52.15636 67.32306) (width 1.70688) (layer F.Cu) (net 1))
 (segment (start 52.18684 67.29258) (end 52.18684 63.84798) (width 1.70688) (layer F.Cu) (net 1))
 (segment (start 52.15636 68.29806) (end 53.5432 69.6849) (width 1.70688) (layer F.Cu) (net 1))
 (segment (start 53.5432 69.6849) (end 58.65876 69.6849) (width 1.70688) (layer F.Cu) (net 1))
 (segment (start 59.84494 68.49872) (end 58.65876 69.6849) (width 1.70688) (layer F.Cu) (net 1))
 (segment (start 59.84494 63.44732) (end 59.84494 68.49872) (width 1.70688) (layer F.Cu) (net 1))
 (segment (start 49.403 32.6136) (end 50.378 32.6136) (width 1.70688) (layer F.Cu) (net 14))
 (segment (start 57.5564 29.1084) (end 57.5564 24.3332) (width 1.70688) (layer F.Cu) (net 14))
 (segment (start 49.403 32.6136) (end 54.0512 32.6136) (width 1.70688) (layer F.Cu) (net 14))
 (segment (start 54.0512 32.6136) (end 57.5564 29.1084) (width 1.70688) (layer F.Cu) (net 14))
 (segment (start 49.3776 32.639) (end 49.403 32.6136) (width 1.70688) (layer F.Cu) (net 14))
 (segment (start 49.3776 36.5855) (end 49.3776 32.639) (width 1.70688) (layer F.Cu) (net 14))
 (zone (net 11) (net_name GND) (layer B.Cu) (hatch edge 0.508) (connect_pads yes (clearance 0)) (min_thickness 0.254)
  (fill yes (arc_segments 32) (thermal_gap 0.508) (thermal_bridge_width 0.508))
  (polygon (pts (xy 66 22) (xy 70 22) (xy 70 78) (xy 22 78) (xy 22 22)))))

